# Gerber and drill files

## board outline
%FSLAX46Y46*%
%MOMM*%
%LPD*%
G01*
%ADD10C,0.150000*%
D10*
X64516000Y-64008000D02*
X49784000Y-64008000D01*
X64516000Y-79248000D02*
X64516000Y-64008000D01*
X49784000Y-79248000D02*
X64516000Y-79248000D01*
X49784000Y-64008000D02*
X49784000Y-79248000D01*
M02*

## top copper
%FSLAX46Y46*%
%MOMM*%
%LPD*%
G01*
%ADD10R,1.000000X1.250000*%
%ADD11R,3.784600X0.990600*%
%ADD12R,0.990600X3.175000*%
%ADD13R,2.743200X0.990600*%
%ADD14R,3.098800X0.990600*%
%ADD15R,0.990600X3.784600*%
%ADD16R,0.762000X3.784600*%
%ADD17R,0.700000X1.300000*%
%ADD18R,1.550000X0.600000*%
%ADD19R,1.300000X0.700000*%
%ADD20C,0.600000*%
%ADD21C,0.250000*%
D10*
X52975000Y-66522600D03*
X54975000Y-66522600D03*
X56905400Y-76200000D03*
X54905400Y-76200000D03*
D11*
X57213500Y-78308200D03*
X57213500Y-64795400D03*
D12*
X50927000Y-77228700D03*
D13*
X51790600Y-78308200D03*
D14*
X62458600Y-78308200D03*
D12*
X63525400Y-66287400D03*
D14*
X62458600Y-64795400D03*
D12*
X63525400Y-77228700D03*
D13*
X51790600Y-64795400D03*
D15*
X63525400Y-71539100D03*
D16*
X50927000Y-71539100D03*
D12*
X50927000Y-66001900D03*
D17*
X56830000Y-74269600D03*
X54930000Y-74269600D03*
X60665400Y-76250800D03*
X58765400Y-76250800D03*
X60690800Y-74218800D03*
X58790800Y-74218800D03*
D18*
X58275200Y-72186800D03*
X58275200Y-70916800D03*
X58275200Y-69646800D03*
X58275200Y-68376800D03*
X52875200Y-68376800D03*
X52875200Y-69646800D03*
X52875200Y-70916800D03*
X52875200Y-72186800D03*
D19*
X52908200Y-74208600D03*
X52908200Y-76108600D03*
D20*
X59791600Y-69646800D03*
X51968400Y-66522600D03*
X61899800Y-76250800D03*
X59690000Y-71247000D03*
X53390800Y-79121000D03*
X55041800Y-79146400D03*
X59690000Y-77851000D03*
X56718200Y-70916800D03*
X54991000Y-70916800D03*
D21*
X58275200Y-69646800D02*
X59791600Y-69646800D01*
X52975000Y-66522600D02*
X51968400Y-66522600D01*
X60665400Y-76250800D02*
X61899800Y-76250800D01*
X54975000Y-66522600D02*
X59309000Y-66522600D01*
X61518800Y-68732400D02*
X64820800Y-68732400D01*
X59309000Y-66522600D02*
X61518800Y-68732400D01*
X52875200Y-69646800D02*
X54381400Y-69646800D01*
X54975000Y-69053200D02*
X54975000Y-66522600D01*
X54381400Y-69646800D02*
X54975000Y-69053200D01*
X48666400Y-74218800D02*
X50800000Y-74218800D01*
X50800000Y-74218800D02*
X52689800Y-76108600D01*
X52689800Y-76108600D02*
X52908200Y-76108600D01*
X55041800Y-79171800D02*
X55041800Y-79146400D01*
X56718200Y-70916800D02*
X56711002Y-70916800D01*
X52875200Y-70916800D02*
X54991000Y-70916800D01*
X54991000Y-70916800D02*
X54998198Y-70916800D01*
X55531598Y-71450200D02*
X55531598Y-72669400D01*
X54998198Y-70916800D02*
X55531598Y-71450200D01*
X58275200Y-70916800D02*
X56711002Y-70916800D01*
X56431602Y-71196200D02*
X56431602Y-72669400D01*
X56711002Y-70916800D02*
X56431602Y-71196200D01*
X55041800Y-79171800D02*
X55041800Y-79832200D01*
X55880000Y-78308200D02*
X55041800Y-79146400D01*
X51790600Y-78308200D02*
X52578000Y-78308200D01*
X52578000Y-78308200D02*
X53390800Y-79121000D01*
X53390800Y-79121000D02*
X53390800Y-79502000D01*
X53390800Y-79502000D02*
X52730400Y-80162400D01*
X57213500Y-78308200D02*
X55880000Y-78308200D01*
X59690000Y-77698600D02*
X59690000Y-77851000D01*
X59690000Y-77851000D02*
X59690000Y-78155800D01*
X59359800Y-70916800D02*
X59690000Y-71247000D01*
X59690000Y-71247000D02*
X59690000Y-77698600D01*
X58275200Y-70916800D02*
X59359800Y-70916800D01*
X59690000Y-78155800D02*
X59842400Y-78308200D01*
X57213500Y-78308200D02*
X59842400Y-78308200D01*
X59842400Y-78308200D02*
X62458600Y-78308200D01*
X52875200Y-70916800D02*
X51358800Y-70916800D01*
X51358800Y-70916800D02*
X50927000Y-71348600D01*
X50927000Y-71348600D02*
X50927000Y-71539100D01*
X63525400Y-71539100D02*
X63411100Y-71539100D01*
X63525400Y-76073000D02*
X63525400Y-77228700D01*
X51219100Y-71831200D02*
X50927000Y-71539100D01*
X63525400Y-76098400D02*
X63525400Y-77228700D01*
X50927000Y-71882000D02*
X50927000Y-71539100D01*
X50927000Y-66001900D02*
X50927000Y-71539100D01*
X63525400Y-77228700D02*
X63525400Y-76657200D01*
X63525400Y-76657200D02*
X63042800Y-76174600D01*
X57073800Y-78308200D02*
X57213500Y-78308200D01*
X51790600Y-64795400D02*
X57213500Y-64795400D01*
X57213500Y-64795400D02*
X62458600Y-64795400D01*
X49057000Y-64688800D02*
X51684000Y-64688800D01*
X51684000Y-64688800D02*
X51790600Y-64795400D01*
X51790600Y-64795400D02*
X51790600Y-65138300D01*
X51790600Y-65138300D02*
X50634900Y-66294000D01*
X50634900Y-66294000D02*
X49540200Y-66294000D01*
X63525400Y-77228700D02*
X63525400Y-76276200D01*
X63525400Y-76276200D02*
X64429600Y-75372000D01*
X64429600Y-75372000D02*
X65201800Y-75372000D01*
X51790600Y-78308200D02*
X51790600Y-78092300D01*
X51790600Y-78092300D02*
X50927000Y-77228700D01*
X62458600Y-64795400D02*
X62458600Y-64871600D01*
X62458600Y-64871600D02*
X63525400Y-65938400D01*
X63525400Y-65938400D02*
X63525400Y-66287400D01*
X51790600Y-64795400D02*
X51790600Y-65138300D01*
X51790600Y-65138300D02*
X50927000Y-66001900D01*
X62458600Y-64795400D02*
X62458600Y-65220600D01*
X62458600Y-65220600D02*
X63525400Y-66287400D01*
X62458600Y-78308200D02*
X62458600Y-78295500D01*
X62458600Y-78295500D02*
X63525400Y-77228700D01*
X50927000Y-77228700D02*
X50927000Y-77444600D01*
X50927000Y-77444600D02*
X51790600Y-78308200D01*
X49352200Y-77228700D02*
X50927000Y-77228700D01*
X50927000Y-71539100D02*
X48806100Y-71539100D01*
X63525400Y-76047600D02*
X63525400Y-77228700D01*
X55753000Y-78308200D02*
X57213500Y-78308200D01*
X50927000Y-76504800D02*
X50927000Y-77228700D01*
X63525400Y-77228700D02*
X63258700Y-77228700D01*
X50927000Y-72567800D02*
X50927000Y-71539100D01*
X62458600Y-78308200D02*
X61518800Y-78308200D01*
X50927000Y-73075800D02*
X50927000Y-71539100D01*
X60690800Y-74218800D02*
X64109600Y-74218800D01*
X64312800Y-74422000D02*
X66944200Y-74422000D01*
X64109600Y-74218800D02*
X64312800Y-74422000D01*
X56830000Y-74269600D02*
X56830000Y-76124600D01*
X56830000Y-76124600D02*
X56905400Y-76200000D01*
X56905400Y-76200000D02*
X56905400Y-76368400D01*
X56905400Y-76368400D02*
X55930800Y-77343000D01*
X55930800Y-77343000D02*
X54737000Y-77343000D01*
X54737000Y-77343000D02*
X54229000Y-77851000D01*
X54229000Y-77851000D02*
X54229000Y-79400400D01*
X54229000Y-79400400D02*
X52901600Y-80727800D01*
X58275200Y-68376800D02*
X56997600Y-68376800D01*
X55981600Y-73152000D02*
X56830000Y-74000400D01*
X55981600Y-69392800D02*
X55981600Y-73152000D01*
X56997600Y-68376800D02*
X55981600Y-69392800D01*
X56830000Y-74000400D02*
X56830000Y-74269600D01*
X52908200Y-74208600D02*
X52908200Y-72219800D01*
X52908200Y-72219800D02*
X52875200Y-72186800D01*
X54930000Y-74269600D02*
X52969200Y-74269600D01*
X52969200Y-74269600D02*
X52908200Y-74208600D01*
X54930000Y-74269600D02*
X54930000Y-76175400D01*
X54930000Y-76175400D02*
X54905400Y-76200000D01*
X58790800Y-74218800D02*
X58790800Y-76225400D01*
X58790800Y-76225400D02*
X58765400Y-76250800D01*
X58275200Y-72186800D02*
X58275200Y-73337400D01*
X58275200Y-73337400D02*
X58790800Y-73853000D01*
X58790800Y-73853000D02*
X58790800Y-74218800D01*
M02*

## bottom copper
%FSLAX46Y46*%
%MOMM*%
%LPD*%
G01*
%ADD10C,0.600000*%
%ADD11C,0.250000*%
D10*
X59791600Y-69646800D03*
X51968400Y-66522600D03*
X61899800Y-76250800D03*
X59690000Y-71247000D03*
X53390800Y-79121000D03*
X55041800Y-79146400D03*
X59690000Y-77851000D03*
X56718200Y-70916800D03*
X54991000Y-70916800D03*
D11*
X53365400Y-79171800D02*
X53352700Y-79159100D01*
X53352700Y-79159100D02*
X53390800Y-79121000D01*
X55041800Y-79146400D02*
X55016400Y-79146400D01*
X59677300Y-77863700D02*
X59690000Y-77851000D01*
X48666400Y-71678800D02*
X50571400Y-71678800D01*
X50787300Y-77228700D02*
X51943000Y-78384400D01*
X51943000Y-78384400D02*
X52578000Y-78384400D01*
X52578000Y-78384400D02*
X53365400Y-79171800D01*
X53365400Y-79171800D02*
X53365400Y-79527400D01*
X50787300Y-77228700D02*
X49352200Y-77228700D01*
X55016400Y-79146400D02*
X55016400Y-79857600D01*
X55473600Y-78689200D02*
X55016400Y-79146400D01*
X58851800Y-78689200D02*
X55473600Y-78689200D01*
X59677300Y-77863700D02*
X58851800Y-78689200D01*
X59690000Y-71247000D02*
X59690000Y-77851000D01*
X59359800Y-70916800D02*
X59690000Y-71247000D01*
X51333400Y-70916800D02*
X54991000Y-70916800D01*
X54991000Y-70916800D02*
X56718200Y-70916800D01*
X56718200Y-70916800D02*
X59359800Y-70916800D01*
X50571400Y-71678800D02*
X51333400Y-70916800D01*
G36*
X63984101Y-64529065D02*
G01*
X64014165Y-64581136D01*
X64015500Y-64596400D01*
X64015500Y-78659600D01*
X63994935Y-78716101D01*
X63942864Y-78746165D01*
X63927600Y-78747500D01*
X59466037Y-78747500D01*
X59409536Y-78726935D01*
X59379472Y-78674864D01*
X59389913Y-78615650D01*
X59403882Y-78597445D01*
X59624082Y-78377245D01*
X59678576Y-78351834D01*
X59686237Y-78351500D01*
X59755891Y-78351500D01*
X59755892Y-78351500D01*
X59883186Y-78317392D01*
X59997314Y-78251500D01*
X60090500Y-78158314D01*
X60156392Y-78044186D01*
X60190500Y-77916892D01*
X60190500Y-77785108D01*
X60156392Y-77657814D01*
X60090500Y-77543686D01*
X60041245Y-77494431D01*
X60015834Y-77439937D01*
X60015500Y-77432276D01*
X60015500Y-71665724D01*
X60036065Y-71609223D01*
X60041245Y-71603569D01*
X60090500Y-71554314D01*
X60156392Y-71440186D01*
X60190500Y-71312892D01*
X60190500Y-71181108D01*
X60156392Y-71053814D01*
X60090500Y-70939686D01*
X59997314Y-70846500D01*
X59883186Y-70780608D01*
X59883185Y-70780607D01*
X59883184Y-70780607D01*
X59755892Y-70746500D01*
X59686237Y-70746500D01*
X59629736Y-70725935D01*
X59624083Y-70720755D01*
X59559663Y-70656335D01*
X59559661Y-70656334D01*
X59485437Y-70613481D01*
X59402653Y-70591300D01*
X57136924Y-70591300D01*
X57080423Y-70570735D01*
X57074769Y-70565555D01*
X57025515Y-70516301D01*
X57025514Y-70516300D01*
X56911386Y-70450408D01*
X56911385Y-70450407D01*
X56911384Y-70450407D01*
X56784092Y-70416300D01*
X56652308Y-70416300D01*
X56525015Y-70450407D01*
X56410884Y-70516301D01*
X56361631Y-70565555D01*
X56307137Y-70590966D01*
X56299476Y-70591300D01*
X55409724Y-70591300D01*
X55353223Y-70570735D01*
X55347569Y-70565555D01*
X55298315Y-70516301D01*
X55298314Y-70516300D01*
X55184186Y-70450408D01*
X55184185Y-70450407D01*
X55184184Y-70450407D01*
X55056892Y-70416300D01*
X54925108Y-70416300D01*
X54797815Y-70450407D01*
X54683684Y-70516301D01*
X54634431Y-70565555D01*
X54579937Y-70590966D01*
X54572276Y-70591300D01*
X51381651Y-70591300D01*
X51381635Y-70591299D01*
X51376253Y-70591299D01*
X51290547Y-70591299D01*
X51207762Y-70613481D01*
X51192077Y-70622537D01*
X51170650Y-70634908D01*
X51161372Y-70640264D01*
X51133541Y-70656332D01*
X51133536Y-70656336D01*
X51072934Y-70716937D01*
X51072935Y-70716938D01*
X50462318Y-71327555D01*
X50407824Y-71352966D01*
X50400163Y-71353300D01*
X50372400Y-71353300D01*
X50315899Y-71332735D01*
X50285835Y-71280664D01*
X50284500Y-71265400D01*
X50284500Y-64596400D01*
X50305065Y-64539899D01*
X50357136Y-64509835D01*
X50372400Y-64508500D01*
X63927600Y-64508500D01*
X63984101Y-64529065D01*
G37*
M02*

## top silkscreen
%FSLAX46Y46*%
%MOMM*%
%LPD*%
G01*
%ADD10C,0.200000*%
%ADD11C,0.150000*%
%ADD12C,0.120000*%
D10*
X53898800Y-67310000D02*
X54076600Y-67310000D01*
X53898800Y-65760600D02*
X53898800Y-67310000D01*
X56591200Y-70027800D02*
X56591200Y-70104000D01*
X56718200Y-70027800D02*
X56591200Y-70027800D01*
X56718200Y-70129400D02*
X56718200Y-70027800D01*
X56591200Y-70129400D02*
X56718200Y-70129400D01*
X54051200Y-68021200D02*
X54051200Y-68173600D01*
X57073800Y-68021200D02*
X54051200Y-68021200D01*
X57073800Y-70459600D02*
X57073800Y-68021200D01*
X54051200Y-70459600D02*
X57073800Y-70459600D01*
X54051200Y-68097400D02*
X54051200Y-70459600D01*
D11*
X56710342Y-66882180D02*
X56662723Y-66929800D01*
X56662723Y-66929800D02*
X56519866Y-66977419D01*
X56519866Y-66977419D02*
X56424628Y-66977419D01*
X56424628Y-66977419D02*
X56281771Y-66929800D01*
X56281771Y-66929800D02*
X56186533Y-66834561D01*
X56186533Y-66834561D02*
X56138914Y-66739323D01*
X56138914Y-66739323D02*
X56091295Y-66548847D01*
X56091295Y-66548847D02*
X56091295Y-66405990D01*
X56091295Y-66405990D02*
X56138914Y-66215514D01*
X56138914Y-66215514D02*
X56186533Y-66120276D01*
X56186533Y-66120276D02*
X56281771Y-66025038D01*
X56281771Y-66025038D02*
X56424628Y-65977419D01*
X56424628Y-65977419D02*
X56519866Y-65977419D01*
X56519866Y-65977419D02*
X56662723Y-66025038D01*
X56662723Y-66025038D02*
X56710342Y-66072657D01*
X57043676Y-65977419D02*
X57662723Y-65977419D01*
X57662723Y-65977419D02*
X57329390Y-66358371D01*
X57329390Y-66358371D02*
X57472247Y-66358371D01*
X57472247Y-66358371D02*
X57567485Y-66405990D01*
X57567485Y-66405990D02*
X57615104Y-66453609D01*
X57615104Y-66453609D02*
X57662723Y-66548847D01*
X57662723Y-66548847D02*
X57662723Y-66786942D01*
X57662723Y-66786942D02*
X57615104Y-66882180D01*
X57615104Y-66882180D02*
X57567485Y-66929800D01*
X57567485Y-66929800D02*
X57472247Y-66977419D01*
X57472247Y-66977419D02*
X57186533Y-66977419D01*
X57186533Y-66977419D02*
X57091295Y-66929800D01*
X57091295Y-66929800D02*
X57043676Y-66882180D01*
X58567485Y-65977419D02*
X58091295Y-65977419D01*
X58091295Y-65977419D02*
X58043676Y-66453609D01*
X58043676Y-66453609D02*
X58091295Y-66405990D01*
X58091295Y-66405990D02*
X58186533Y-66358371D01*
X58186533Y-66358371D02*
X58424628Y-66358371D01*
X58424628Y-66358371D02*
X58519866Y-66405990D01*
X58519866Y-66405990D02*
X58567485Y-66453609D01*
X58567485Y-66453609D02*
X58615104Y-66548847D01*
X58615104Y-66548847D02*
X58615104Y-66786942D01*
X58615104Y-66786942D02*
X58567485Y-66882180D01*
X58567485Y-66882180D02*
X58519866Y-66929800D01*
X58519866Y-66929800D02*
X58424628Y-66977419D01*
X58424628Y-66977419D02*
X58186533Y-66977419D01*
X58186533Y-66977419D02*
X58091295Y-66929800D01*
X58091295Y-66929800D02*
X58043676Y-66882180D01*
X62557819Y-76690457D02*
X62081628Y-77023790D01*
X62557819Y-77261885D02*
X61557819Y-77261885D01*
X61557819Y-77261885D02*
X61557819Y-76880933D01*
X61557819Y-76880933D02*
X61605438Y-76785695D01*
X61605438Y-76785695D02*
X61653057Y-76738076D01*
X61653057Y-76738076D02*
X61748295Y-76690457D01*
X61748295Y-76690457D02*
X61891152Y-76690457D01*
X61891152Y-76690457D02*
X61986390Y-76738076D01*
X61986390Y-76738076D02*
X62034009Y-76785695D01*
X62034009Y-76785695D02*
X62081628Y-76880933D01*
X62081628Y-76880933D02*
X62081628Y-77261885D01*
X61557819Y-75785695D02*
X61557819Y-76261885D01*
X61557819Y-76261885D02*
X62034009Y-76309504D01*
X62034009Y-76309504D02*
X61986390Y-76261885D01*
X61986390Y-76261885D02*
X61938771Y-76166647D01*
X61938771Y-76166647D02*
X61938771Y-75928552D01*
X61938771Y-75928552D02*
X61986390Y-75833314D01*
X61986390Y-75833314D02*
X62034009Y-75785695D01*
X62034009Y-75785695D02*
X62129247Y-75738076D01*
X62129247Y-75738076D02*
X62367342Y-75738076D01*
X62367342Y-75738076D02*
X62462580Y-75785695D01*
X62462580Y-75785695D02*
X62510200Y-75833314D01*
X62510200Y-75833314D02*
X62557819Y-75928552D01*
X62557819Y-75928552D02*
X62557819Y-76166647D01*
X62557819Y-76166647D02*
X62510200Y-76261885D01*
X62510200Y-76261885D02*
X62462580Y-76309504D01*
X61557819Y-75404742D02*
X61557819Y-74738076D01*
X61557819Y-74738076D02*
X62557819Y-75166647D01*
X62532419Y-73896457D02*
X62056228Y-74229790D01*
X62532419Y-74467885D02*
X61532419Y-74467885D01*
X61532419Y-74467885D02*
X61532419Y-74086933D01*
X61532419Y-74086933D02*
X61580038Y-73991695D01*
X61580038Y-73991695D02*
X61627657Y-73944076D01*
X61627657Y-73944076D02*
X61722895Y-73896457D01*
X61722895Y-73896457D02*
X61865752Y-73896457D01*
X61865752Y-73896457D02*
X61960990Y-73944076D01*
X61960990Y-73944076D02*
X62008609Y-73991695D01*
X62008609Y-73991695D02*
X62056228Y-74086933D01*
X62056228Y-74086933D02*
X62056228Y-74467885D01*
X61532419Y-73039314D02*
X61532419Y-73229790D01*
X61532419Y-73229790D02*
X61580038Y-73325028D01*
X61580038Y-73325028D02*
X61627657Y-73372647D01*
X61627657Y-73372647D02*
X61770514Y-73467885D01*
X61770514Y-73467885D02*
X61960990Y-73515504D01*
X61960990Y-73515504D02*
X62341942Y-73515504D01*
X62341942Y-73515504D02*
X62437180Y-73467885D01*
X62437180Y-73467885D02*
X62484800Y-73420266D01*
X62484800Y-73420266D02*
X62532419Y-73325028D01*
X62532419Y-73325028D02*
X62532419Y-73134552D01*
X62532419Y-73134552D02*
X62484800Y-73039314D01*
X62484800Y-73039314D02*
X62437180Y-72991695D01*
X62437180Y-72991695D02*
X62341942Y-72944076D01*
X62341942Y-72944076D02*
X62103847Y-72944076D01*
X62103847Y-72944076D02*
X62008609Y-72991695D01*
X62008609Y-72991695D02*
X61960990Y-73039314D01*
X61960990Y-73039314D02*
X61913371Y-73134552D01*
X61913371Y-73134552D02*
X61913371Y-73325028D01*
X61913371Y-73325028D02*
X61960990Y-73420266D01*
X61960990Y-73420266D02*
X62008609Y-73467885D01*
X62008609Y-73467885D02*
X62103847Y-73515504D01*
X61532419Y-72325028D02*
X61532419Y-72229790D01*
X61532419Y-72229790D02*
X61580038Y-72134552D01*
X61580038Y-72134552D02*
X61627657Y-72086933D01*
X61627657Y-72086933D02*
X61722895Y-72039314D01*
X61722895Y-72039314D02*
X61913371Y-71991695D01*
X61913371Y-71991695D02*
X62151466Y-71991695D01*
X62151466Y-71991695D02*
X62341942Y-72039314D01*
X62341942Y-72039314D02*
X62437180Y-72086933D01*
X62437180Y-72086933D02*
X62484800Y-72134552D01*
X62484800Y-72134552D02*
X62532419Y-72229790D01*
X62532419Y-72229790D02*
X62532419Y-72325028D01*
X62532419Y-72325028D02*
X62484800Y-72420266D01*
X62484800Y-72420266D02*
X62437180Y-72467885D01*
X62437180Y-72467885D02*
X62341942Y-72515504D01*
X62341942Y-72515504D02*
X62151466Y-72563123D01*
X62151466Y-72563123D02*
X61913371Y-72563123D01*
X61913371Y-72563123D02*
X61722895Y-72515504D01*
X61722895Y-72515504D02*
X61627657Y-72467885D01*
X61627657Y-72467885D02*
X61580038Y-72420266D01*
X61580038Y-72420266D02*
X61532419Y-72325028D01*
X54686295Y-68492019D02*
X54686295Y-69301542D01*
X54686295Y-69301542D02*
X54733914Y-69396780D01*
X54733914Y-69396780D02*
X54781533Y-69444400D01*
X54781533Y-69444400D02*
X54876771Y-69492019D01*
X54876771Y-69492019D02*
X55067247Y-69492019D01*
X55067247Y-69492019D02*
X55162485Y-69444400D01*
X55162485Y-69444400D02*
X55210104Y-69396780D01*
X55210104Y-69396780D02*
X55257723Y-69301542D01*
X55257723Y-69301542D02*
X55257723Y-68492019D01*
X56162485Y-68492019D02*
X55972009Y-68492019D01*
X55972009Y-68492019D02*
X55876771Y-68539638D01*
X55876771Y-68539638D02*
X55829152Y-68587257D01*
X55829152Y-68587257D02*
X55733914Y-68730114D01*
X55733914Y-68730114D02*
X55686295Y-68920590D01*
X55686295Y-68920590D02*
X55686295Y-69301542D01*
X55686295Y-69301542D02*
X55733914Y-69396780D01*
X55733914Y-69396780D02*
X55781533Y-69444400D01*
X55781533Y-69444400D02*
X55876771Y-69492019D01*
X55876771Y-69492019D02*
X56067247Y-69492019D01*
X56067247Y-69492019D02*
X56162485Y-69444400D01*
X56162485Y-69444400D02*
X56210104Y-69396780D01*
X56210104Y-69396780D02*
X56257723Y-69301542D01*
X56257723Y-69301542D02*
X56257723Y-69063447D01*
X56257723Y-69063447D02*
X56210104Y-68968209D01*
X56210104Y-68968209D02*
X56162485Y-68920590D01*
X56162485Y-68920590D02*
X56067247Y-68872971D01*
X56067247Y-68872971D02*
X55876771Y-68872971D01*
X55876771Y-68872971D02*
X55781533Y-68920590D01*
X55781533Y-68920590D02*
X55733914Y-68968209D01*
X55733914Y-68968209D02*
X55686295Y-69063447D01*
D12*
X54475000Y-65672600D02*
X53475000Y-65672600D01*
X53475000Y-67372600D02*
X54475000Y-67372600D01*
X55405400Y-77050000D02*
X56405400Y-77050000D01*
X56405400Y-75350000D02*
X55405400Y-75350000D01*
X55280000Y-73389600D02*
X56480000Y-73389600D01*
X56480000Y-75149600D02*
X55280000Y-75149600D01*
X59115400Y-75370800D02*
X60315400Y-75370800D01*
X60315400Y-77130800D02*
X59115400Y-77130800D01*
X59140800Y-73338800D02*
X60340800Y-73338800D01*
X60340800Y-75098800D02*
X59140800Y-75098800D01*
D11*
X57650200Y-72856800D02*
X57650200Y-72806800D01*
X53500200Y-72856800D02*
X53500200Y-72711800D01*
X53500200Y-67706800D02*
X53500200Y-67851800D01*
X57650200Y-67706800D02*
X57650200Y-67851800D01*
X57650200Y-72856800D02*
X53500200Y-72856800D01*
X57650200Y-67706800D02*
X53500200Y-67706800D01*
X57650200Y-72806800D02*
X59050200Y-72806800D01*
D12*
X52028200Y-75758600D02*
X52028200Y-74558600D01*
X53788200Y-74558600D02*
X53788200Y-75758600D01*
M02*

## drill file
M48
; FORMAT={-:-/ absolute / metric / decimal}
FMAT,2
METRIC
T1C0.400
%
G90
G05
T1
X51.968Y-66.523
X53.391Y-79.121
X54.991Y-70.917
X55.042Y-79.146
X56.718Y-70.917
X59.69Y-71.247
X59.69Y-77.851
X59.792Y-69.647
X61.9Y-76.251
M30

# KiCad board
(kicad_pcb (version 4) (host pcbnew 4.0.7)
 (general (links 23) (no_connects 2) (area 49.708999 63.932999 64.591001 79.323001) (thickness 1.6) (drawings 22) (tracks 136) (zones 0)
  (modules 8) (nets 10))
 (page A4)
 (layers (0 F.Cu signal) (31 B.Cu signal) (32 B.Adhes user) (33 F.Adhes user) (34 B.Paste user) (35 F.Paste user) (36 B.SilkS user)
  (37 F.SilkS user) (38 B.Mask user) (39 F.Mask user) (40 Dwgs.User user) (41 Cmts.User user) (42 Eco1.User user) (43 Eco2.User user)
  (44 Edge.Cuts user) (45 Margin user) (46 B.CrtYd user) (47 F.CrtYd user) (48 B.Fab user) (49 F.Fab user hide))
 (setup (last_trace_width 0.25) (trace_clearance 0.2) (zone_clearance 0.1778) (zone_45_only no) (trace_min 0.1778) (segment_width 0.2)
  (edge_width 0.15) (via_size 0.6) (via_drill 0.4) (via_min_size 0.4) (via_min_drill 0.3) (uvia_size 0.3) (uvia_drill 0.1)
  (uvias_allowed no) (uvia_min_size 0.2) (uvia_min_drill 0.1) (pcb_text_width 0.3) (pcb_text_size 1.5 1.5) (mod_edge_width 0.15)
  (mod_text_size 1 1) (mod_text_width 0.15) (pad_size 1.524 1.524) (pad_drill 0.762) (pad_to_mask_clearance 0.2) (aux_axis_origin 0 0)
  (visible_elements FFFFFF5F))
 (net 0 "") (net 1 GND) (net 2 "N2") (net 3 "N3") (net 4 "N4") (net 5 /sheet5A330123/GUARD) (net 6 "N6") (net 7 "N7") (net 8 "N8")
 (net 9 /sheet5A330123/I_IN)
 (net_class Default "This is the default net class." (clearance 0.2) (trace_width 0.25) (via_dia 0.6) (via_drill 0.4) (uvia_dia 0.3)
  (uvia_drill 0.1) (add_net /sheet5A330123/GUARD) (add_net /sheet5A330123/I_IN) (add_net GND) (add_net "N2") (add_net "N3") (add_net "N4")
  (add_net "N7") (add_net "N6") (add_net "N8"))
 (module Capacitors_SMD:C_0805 (layer F.Cu) (at 53.975 66.5226)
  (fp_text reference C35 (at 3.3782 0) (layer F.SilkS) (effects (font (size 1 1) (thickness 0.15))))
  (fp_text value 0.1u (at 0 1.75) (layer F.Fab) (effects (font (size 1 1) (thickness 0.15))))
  (fp_line (start 0.5 -0.85) (end -0.5 -0.85) (layer F.SilkS) (width 0.12))
  (fp_line (start -0.5 0.85) (end 0.5 0.85) (layer F.SilkS) (width 0.12))
  (pad 1 smd rect (at -1 0) (size 1 1.25) (layers F.Cu F.Paste F.Mask) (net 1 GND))
  (pad 2 smd rect (at 1 0) (size 1 1.25) (layers F.Cu F.Paste F.Mask) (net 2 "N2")))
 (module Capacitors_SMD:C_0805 (layer F.Cu) (at 55.9054 76.2 180)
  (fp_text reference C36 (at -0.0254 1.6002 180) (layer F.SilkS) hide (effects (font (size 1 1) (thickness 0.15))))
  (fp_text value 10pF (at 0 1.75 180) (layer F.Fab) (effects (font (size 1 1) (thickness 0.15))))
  (fp_line (start 0.5 -0.85) (end -0.5 -0.85) (layer F.SilkS) (width 0.12))
  (fp_line (start -0.5 0.85) (end 0.5 0.85) (layer F.SilkS) (width 0.12))
  (pad 1 smd rect (at -1 0 180) (size 1 1.25) (layers F.Cu F.Paste F.Mask) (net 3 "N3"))
  (pad 2 smd rect (at 1 0 180) (size 1 1.25) (layers F.Cu F.Paste F.Mask) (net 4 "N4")))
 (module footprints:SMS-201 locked (layer F.Cu) (at 50.419 64.2874)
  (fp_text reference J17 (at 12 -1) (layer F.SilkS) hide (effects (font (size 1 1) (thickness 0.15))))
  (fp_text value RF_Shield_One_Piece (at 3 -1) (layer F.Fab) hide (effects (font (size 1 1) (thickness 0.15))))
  (pad 1 smd rect (at 6.7945 14.0208 90) (size 0.9906 3.7846) (layers F.Cu F.Paste F.Mask) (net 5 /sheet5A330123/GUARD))
  (pad 1 smd rect (at 6.7945 0.508 90) (size 0.9906 3.7846) (layers F.Cu F.Paste F.Mask) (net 5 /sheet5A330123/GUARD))
  (pad 1 smd rect (at 0.508 12.9413 180) (size 0.9906 3.175) (layers F.Cu F.Paste F.Mask) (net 5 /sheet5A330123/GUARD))
  (pad 1 smd rect (at 1.3716 14.0208) (size 2.7432 0.9906) (layers F.Cu F.Paste F.Mask) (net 5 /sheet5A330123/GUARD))
  (pad 1 smd rect (at 12.0396 14.0208 270) (size 0.9906 3.0988) (layers F.Cu F.Paste F.Mask) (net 5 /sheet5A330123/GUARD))
  (pad 1 smd rect (at 13.1064 2 180) (size 0.9906 3.175) (layers F.Cu F.Paste F.Mask) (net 5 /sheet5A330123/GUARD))
  (pad 1 smd rect (at 12.0396 0.508 270) (size 0.9906 3.0988) (layers F.Cu F.Paste F.Mask) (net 5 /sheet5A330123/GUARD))
  (pad 1 smd rect (at 13.1064 12.9413) (size 0.9906 3.175) (layers F.Cu F.Paste F.Mask) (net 5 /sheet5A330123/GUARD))
  (pad 1 smd rect (at 1.3716 0.508 90) (size 0.9906 2.7432) (layers F.Cu F.Paste F.Mask) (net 5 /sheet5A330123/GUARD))
  (pad 1 smd rect (at 13.1064 7.2517) (size 0.9906 3.7846) (layers F.Cu F.Paste F.Mask) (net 5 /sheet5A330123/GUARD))
  (pad 1 smd rect (at 0.508 7.2517) (size 0.762 3.7846) (layers F.Cu F.Paste F.Mask) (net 5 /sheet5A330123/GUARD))
  (pad 1 smd rect (at 0.508 1.7145) (size 0.9906 3.175) (layers F.Cu F.Paste F.Mask) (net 5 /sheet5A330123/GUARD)))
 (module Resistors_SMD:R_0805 (layer F.Cu) (at 55.88 74.2696 180)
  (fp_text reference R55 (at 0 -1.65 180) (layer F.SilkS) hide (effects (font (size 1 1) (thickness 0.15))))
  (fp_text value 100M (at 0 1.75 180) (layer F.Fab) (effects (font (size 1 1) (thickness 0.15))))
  (fp_line (start 0.6 0.88) (end -0.6 0.88) (layer F.SilkS) (width 0.12))
  (fp_line (start -0.6 -0.88) (end 0.6 -0.88) (layer F.SilkS) (width 0.12))
  (pad 1 smd rect (at -0.95 0 180) (size 0.7 1.3) (layers F.Cu F.Paste F.Mask) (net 3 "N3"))
  (pad 2 smd rect (at 0.95 0 180) (size 0.7 1.3) (layers F.Cu F.Paste F.Mask) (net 4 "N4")))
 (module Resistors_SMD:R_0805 (layer F.Cu) (at 59.7154 76.2508 180)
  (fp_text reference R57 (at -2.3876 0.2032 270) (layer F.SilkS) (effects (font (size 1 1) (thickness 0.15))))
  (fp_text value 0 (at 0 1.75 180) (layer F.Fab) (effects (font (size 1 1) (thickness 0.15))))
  (fp_line (start 0.6 0.88) (end -0.6 0.88) (layer F.SilkS) (width 0.12))
  (fp_line (start -0.6 -0.88) (end 0.6 -0.88) (layer F.SilkS) (width 0.12))
  (pad 1 smd rect (at -0.95 0 180) (size 0.7 1.3) (layers F.Cu F.Paste F.Mask) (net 1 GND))
  (pad 2 smd rect (at 0.95 0 180) (size 0.7 1.3) (layers F.Cu F.Paste F.Mask) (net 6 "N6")))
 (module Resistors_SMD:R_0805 (layer F.Cu) (at 59.7408 74.2188 180)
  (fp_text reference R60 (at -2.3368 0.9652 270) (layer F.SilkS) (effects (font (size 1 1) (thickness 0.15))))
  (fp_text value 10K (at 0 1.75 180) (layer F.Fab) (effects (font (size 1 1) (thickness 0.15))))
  (fp_line (start 0.6 0.88) (end -0.6 0.88) (layer F.SilkS) (width 0.12))
  (fp_line (start -0.6 -0.88) (end 0.6 -0.88) (layer F.SilkS) (width 0.12))
  (pad 1 smd rect (at -0.95 0 180) (size 0.7 1.3) (layers F.Cu F.Paste F.Mask) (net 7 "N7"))
  (pad 2 smd rect (at 0.95 0 180) (size 0.7 1.3) (layers F.Cu F.Paste F.Mask) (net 6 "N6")))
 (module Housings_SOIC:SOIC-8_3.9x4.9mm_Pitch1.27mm (layer F.Cu) (at 55.5752 70.2818 180)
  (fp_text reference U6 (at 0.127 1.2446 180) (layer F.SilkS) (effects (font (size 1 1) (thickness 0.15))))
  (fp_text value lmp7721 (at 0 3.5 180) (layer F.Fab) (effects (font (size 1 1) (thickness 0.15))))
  (fp_line (start -2.075 -2.575) (end -2.075 -2.525) (layer F.SilkS) (width 0.15))
  (fp_line (start 2.075 -2.575) (end 2.075 -2.43) (layer F.SilkS) (width 0.15))
  (fp_line (start 2.075 2.575) (end 2.075 2.43) (layer F.SilkS) (width 0.15))
  (fp_line (start -2.075 2.575) (end -2.075 2.43) (layer F.SilkS) (width 0.15))
  (fp_line (start -2.075 -2.575) (end 2.075 -2.575) (layer F.SilkS) (width 0.15))
  (fp_line (start -2.075 2.575) (end 2.075 2.575) (layer F.SilkS) (width 0.15))
  (fp_line (start -2.075 -2.525) (end -3.475 -2.525) (layer F.SilkS) (width 0.15))
  (pad 1 smd rect (at -2.7 -1.905 180) (size 1.55 0.6) (layers F.Cu F.Paste F.Mask) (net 6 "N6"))
  (pad 2 smd rect (at -2.7 -0.635 180) (size 1.55 0.6) (layers F.Cu F.Paste F.Mask) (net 5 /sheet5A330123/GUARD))
  (pad 3 smd rect (at -2.7 0.635 180) (size 1.55 0.6) (layers F.Cu F.Paste F.Mask) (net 1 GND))
  (pad 4 smd rect (at -2.7 1.905 180) (size 1.55 0.6) (layers F.Cu F.Paste F.Mask) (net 3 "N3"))
  (pad 5 smd rect (at 2.7 1.905 180) (size 1.55 0.6) (layers F.Cu F.Paste F.Mask) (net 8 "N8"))
  (pad 6 smd rect (at 2.7 0.635 180) (size 1.55 0.6) (layers F.Cu F.Paste F.Mask) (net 2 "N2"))
  (pad 7 smd rect (at 2.7 -0.635 180) (size 1.55 0.6) (layers F.Cu F.Paste F.Mask) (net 5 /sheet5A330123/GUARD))
  (pad 8 smd rect (at 2.7 -1.905 180) (size 1.55 0.6) (layers F.Cu F.Paste F.Mask) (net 4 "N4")))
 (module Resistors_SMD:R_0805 (layer F.Cu) (at 52.9082 75.1586 270)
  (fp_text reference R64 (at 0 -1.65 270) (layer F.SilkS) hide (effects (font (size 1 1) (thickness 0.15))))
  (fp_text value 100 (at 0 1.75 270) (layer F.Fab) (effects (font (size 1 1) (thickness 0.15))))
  (fp_line (start 0.6 0.88) (end -0.6 0.88) (layer F.SilkS) (width 0.12))
  (fp_line (start -0.6 -0.88) (end 0.6 -0.88) (layer F.SilkS) (width 0.12))
  (pad 1 smd rect (at -0.95 0 270) (size 0.7 1.3) (layers F.Cu F.Paste F.Mask) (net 4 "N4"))
  (pad 2 smd rect (at 0.95 0 270) (size 0.7 1.3) (layers F.Cu F.Paste F.Mask) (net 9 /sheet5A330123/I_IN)))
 (gr_line (start 64.516 64.008) (end 49.784 64.008) (angle 90) (layer Edge.Cuts) (width 0.15))
 (gr_line (start 64.516 79.248) (end 64.516 64.008) (angle 90) (layer Edge.Cuts) (width 0.15))
 (gr_line (start 49.784 79.248) (end 64.516 79.248) (angle 90) (layer Edge.Cuts) (width 0.15))
 (gr_line (start 49.784 64.008) (end 49.784 79.248) (angle 90) (layer Edge.Cuts) (width 0.15))
 (gr_line (start 53.8988 67.31) (end 54.0766 67.31) (angle 90) (layer F.SilkS) (width 0.2))
 (gr_line (start 53.8988 65.7606) (end 53.8988 67.31) (angle 90) (layer F.SilkS) (width 0.2))
 (gr_line (start 56.5912 70.0278) (end 56.5912 70.104) (angle 90) (layer F.SilkS) (width 0.2))
 (gr_line (start 56.7182 70.0278) (end 56.5912 70.0278) (angle 90) (layer F.SilkS) (width 0.2))
 (gr_line (start 56.7182 70.1294) (end 56.7182 70.0278) (angle 90) (layer F.SilkS) (width 0.2))
 (gr_line (start 56.5912 70.1294) (end 56.7182 70.1294) (angle 90) (layer F.SilkS) (width 0.2))
 (gr_line (start 54.0512 68.0212) (end 54.0512 68.1736) (angle 90) (layer F.SilkS) (width 0.2))
 (gr_line (start 57.0738 68.0212) (end 54.0512 68.0212) (angle 90) (layer F.SilkS) (width 0.2))
 (gr_line (start 57.0738 70.4596) (end 57.0738 68.0212) (angle 90) (layer F.SilkS) (width 0.2))
 (gr_line (start 54.0512 70.4596) (end 57.0738 70.4596) (angle 90) (layer F.SilkS) (width 0.2))
 (gr_line (start 54.0512 68.0974) (end 54.0512 70.4596) (angle 90) (layer F.SilkS) (width 0.2))
 (segment (start 58.2752 69.6468) (end 59.7916 69.6468) (width 0.25) (layer F.Cu) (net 1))
 (via (at 59.7916 69.6468) (size 0.6) (drill 0.4) (layers F.Cu B.Cu) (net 1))
 (segment (start 52.975 66.5226) (end 51.9684 66.5226) (width 0.25) (layer F.Cu) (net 1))
 (via (at 51.9684 66.5226) (size 0.6) (drill 0.4) (layers F.Cu B.Cu) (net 1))
 (segment (start 60.6654 76.2508) (end 61.8998 76.2508) (width 0.25) (layer F.Cu) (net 1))
 (via (at 61.8998 76.2508) (size 0.6) (drill 0.4) (layers F.Cu B.Cu) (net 1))
 (segment (start 54.975 66.5226) (end 59.309 66.5226) (width 0.25) (layer F.Cu) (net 2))
 (segment (start 61.5188 68.7324) (end 64.8208 68.7324) (width 0.25) (layer F.Cu) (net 2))
 (segment (start 59.309 66.5226) (end 61.5188 68.7324) (width 0.25) (layer F.Cu) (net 2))
 (segment (start 52.8752 69.6468) (end 54.3814 69.6468) (width 0.25) (layer F.Cu) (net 2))
 (segment (start 54.975 69.0532) (end 54.975 66.5226) (width 0.25) (layer F.Cu) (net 2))
 (segment (start 54.3814 69.6468) (end 54.975 69.0532) (width 0.25) (layer F.Cu) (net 2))
 (segment (start 48.6664 74.2188) (end 50.8 74.2188) (width 0.25) (layer F.Cu) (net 9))
 (segment (start 50.8 74.2188) (end 52.6898 76.1086) (width 0.25) (layer F.Cu) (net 9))
 (segment (start 52.6898 76.1086) (end 52.9082 76.1086) (width 0.25) (layer F.Cu) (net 9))
 (via (at 59.69 71.247) (size 0.6) (drill 0.4) (layers F.Cu B.Cu) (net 5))
 (via (at 53.3908 79.121) (size 0.6) (drill 0.4) (layers F.Cu B.Cu) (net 5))
 (segment (start 53.3654 79.1718) (end 53.3527 79.1591) (width 0.25) (layer B.Cu) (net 5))
 (segment (start 53.3527 79.1591) (end 53.3908 79.121) (width 0.25) (layer B.Cu) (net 5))
 (segment (start 55.0418 79.1718) (end 55.0418 79.1464) (width 0.25) (layer F.Cu) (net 5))
 (via (at 55.0418 79.1464) (size 0.6) (drill 0.4) (layers F.Cu B.Cu) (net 5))
 (segment (start 55.0418 79.1464) (end 55.0164 79.1464) (width 0.25) (layer B.Cu) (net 5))
 (segment (start 59.6773 77.8637) (end 59.69 77.851) (width 0.25) (layer B.Cu) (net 5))
 (via (at 59.69 77.851) (size 0.6) (drill 0.4) (layers F.Cu B.Cu) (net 5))
 (via (at 56.7182 70.9168) (size 0.6) (drill 0.4) (layers F.Cu B.Cu) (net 5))
 (segment (start 56.7182 70.9168) (end 56.711002 70.9168) (width 0.25) (layer F.Cu) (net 5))
 (via (at 54.991 70.9168) (size 0.6) (drill 0.4) (layers F.Cu B.Cu) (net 5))
 (segment (start 48.6664 71.6788) (end 50.5714 71.6788) (width 0.25) (layer B.Cu) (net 5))
 (segment (start 50.7873 77.2287) (end 51.943 78.3844) (width 0.25) (layer B.Cu) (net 5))
 (segment (start 51.943 78.3844) (end 52.578 78.3844) (width 0.25) (layer B.Cu) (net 5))
 (segment (start 52.578 78.3844) (end 53.3654 79.1718) (width 0.25) (layer B.Cu) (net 5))
 (segment (start 53.3654 79.1718) (end 53.3654 79.5274) (width 0.25) (layer B.Cu) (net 5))
 (segment (start 50.7873 77.2287) (end 49.3522 77.2287) (width 0.25) (layer B.Cu) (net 5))
 (segment (start 55.0164 79.1464) (end 55.0164 79.8576) (width 0.25) (layer B.Cu) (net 5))
 (segment (start 55.4736 78.6892) (end 55.0164 79.1464) (width 0.25) (layer B.Cu) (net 5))
 (segment (start 58.8518 78.6892) (end 55.4736 78.6892) (width 0.25) (layer B.Cu) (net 5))
 (segment (start 59.6773 77.8637) (end 58.8518 78.6892) (width 0.25) (layer B.Cu) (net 5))
 (segment (start 59.69 71.247) (end 59.69 77.851) (width 0.25) (layer B.Cu) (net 5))
 (segment (start 59.3598 70.9168) (end 59.69 71.247) (width 0.25) (layer B.Cu) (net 5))
 (segment (start 51.3334 70.9168) (end 54.991 70.9168) (width 0.25) (layer B.Cu) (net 5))
 (segment (start 54.991 70.9168) (end 56.7182 70.9168) (width 0.25) (layer B.Cu) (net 5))
 (segment (start 56.7182 70.9168) (end 59.3598 70.9168) (width 0.25) (layer B.Cu) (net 5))
 (segment (start 50.5714 71.6788) (end 51.3334 70.9168) (width 0.25) (layer B.Cu) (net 5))
 (segment (start 52.8752 70.9168) (end 54.991 70.9168) (width 0.25) (layer F.Cu) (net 5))
 (segment (start 54.991 70.9168) (end 54.998198 70.9168) (width 0.25) (layer F.Cu) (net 5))
 (segment (start 55.531598 71.4502) (end 55.531598 72.6694) (width 0.25) (layer F.Cu) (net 5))
 (segment (start 54.998198 70.9168) (end 55.531598 71.4502) (width 0.25) (layer F.Cu) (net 5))
 (segment (start 58.2752 70.9168) (end 56.711002 70.9168) (width 0.25) (layer F.Cu) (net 5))
 (segment (start 56.431602 71.1962) (end 56.431602 72.6694) (width 0.25) (layer F.Cu) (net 5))
 (segment (start 56.711002 70.9168) (end 56.431602 71.1962) (width 0.25) (layer F.Cu) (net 5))
 (segment (start 55.0418 79.1718) (end 55.0418 79.8322) (width 0.25) (layer F.Cu) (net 5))
 (segment (start 55.88 78.3082) (end 55.0418 79.1464) (width 0.25) (layer F.Cu) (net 5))
 (segment (start 51.7906 78.3082) (end 52.578 78.3082) (width 0.25) (layer F.Cu) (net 5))
 (segment (start 52.578 78.3082) (end 53.3908 79.121) (width 0.25) (layer F.Cu) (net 5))
 (segment (start 53.3908 79.121) (end 53.3908 79.502) (width 0.25) (layer F.Cu) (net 5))
 (segment (start 53.3908 79.502) (end 52.7304 80.1624) (width 0.25) (layer F.Cu) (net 5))
 (segment (start 57.2135 78.3082) (end 55.88 78.3082) (width 0.25) (layer F.Cu) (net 5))
 (segment (start 59.69 77.6986) (end 59.69 77.851) (width 0.25) (layer F.Cu) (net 5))
 (segment (start 59.69 77.851) (end 59.69 78.1558) (width 0.25) (layer F.Cu) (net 5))
 (segment (start 59.3598 70.9168) (end 59.69 71.247) (width 0.25) (layer F.Cu) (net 5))
 (segment (start 59.69 71.247) (end 59.69 77.6986) (width 0.25) (layer F.Cu) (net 5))
 (segment (start 58.2752 70.9168) (end 59.3598 70.9168) (width 0.25) (layer F.Cu) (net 5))
 (segment (start 59.69 78.1558) (end 59.8424 78.3082) (width 0.25) (layer F.Cu) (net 5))
 (segment (start 57.2135 78.3082) (end 59.8424 78.3082) (width 0.25) (layer F.Cu) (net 5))
 (segment (start 59.8424 78.3082) (end 62.4586 78.3082) (width 0.25) (layer F.Cu) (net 5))
 (segment (start 52.8752 70.9168) (end 51.3588 70.9168) (width 0.25) (layer F.Cu) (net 5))
 (segment (start 51.3588 70.9168) (end 50.927 71.3486) (width 0.25) (layer F.Cu) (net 5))
 (segment (start 50.927 71.3486) (end 50.927 71.5391) (width 0.25) (layer F.Cu) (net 5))
 (segment (start 63.5254 71.5391) (end 63.4111 71.5391) (width 0.25) (layer F.Cu) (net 5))
 (segment (start 63.5254 76.073) (end 63.5254 77.2287) (width 0.25) (layer F.Cu) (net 5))
 (segment (start 51.2191 71.8312) (end 50.927 71.5391) (width 0.25) (layer F.Cu) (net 5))
 (segment (start 63.5254 76.0984) (end 63.5254 77.2287) (width 0.25) (layer F.Cu) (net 5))
 (segment (start 50.927 71.882) (end 50.927 71.5391) (width 0.25) (layer F.Cu) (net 5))
 (segment (start 50.927 66.0019) (end 50.927 71.5391) (width 0.25) (layer F.Cu) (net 5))
 (segment (start 63.5254 77.2287) (end 63.5254 76.6572) (width 0.25) (layer F.Cu) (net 5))
 (segment (start 63.5254 76.6572) (end 63.0428 76.1746) (width 0.25) (layer F.Cu) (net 5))
 (segment (start 57.0738 78.3082) (end 57.2135 78.3082) (width 0.25) (layer F.Cu) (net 5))
 (segment (start 51.7906 64.7954) (end 57.2135 64.7954) (width 0.25) (layer F.Cu) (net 5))
 (segment (start 57.2135 64.7954) (end 62.4586 64.7954) (width 0.25) (layer F.Cu) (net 5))
 (segment (start 49.057 64.6888) (end 51.684 64.6888) (width 0.25) (layer F.Cu) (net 5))
 (segment (start 51.684 64.6888) (end 51.7906 64.7954) (width 0.25) (layer F.Cu) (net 5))
 (segment (start 51.7906 64.7954) (end 51.7906 65.1383) (width 0.25) (layer F.Cu) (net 5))
 (segment (start 51.7906 65.1383) (end 50.6349 66.294) (width 0.25) (layer F.Cu) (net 5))
 (segment (start 50.6349 66.294) (end 49.5402 66.294) (width 0.25) (layer F.Cu) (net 5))
 (segment (start 63.5254 77.2287) (end 63.5254 76.2762) (width 0.25) (layer F.Cu) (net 5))
 (segment (start 63.5254 76.2762) (end 64.4296 75.372) (width 0.25) (layer F.Cu) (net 5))
 (segment (start 64.4296 75.372) (end 65.2018 75.372) (width 0.25) (layer F.Cu) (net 5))
 (segment (start 51.7906 78.3082) (end 51.7906 78.0923) (width 0.25) (layer F.Cu) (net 5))
 (segment (start 51.7906 78.0923) (end 50.927 77.2287) (width 0.25) (layer F.Cu) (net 5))
 (segment (start 62.4586 64.7954) (end 62.4586 64.8716) (width 0.25) (layer F.Cu) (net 5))
 (segment (start 62.4586 64.8716) (end 63.5254 65.9384) (width 0.25) (layer F.Cu) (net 5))
 (segment (start 63.5254 65.9384) (end 63.5254 66.2874) (width 0.25) (layer F.Cu) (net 5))
 (segment (start 51.7906 64.7954) (end 51.7906 65.1383) (width 0.25) (layer F.Cu) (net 5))
 (segment (start 51.7906 65.1383) (end 50.927 66.0019) (width 0.25) (layer F.Cu) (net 5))
 (segment (start 62.4586 64.7954) (end 62.4586 65.2206) (width 0.25) (layer F.Cu) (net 5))
 (segment (start 62.4586 65.2206) (end 63.5254 66.2874) (width 0.25) (layer F.Cu) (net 5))
 (segment (start 62.4586 78.3082) (end 62.4586 78.2955) (width 0.25) (layer F.Cu) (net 5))
 (segment (start 62.4586 78.2955) (end 63.5254 77.2287) (width 0.25) (layer F.Cu) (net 5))
 (segment (start 50.927 77.2287) (end 50.927 77.4446) (width 0.25) (layer F.Cu) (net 5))
 (segment (start 50.927 77.4446) (end 51.7906 78.3082) (width 0.25) (layer F.Cu) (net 5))
 (segment (start 49.3522 77.2287) (end 50.927 77.2287) (width 0.25) (layer F.Cu) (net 5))
 (segment (start 50.927 71.5391) (end 48.8061 71.5391) (width 0.25) (layer F.Cu) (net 5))
 (segment (start 63.5254 76.0476) (end 63.5254 77.2287) (width 0.25) (layer F.Cu) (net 5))
 (segment (start 55.753 78.3082) (end 57.2135 78.3082) (width 0.25) (layer F.Cu) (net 5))
 (segment (start 50.927 76.5048) (end 50.927 77.2287) (width 0.25) (layer F.Cu) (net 5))
 (segment (start 63.5254 77.2287) (end 63.2587 77.2287) (width 0.25) (layer F.Cu) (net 5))
 (segment (start 50.927 72.5678) (end 50.927 71.5391) (width 0.25) (layer F.Cu) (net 5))
 (segment (start 62.4586 78.3082) (end 61.5188 78.3082) (width 0.25) (layer F.Cu) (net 5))
 (segment (start 50.927 73.0758) (end 50.927 71.5391) (width 0.25) (layer F.Cu) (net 5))
 (segment (start 60.6908 74.2188) (end 64.1096 74.2188) (width 0.25) (layer F.Cu) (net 7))
 (segment (start 64.3128 74.422) (end 66.9442 74.422) (width 0.25) (layer F.Cu) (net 7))
 (segment (start 64.1096 74.2188) (end 64.3128 74.422) (width 0.25) (layer F.Cu) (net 7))
 (segment (start 56.83 74.2696) (end 56.83 76.1246) (width 0.25) (layer F.Cu) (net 3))
 (segment (start 56.83 76.1246) (end 56.9054 76.2) (width 0.25) (layer F.Cu) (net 3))
 (segment (start 56.9054 76.2) (end 56.9054 76.3684) (width 0.25) (layer F.Cu) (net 3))
 (segment (start 56.9054 76.3684) (end 55.9308 77.343) (width 0.25) (layer F.Cu) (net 3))
 (segment (start 55.9308 77.343) (end 54.737 77.343) (width 0.25) (layer F.Cu) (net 3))
 (segment (start 54.737 77.343) (end 54.229 77.851) (width 0.25) (layer F.Cu) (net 3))
 (segment (start 54.229 77.851) (end 54.229 79.4004) (width 0.25) (layer F.Cu) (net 3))
 (segment (start 54.229 79.4004) (end 52.9016 80.7278) (width 0.25) (layer F.Cu) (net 3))
 (segment (start 58.2752 68.3768) (end 56.9976 68.3768) (width 0.25) (layer F.Cu) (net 3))
 (segment (start 55.9816 73.152) (end 56.83 74.0004) (width 0.25) (layer F.Cu) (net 3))
 (segment (start 55.9816 69.3928) (end 55.9816 73.152) (width 0.25) (layer F.Cu) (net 3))
 (segment (start 56.9976 68.3768) (end 55.9816 69.3928) (width 0.25) (layer F.Cu) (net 3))
 (segment (start 56.83 74.0004) (end 56.83 74.2696) (width 0.25) (layer F.Cu) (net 3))
 (segment (start 52.9082 74.2086) (end 52.9082 72.2198) (width 0.25) (layer F.Cu) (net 4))
 (segment (start 52.9082 72.2198) (end 52.8752 72.1868) (width 0.25) (layer F.Cu) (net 4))
 (segment (start 54.93 74.2696) (end 52.9692 74.2696) (width 0.25) (layer F.Cu) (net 4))
 (segment (start 52.9692 74.2696) (end 52.9082 74.2086) (width 0.25) (layer F.Cu) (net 4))
 (segment (start 54.93 74.2696) (end 54.93 76.1754) (width 0.25) (layer F.Cu) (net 4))
 (segment (start 54.93 76.1754) (end 54.9054 76.2) (width 0.25) (layer F.Cu) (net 4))
 (segment (start 58.7908 74.2188) (end 58.7908 76.2254) (width 0.25) (layer F.Cu) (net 6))
 (segment (start 58.7908 76.2254) (end 58.7654 76.2508) (width 0.25) (layer F.Cu) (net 6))
 (segment (start 58.2752 72.1868) (end 58.2752 73.3374) (width 0.25) (layer F.Cu) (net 6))
 (segment (start 58.2752 73.3374) (end 58.7908 73.853) (width 0.25) (layer F.Cu) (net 6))
 (segment (start 58.7908 73.853) (end 58.7908 74.2188) (width 0.25) (layer F.Cu) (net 6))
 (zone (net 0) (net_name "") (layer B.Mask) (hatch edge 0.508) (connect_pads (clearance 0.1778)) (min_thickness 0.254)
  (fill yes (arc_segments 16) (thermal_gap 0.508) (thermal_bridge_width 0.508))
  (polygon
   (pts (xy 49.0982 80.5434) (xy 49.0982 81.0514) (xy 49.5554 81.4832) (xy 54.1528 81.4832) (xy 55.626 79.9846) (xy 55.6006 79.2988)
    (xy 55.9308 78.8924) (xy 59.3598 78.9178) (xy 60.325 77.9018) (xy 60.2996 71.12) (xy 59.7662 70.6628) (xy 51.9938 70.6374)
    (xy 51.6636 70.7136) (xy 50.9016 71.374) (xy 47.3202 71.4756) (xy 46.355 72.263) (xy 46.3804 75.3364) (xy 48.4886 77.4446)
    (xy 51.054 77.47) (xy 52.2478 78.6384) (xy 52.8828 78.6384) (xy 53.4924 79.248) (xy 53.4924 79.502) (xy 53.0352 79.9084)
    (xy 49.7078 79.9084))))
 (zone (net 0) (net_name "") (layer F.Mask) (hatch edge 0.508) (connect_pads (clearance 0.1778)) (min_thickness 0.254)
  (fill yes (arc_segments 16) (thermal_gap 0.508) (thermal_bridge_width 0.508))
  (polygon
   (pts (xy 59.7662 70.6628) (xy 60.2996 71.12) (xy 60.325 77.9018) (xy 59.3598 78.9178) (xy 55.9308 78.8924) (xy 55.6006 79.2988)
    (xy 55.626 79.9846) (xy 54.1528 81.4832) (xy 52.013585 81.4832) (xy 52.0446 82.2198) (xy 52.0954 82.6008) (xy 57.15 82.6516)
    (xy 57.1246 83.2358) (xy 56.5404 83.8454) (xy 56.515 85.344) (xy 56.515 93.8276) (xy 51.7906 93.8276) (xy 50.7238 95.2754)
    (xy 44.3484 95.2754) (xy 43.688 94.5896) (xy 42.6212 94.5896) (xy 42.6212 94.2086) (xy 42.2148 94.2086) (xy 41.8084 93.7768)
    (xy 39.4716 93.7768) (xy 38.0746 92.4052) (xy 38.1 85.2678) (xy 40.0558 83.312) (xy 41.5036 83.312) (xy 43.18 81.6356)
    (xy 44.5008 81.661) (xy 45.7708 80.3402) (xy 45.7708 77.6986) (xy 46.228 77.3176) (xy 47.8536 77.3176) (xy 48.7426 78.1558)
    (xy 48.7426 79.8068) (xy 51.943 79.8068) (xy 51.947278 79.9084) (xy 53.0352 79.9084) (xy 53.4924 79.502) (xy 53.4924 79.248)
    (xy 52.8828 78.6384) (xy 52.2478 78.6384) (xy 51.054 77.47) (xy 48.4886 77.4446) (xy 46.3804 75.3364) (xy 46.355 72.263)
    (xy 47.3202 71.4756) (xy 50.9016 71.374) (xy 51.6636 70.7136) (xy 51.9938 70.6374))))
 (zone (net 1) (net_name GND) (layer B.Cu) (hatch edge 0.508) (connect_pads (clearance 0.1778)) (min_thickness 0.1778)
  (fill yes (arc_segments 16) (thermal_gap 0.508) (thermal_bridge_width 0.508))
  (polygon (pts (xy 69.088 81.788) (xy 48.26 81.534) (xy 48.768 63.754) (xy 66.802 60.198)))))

